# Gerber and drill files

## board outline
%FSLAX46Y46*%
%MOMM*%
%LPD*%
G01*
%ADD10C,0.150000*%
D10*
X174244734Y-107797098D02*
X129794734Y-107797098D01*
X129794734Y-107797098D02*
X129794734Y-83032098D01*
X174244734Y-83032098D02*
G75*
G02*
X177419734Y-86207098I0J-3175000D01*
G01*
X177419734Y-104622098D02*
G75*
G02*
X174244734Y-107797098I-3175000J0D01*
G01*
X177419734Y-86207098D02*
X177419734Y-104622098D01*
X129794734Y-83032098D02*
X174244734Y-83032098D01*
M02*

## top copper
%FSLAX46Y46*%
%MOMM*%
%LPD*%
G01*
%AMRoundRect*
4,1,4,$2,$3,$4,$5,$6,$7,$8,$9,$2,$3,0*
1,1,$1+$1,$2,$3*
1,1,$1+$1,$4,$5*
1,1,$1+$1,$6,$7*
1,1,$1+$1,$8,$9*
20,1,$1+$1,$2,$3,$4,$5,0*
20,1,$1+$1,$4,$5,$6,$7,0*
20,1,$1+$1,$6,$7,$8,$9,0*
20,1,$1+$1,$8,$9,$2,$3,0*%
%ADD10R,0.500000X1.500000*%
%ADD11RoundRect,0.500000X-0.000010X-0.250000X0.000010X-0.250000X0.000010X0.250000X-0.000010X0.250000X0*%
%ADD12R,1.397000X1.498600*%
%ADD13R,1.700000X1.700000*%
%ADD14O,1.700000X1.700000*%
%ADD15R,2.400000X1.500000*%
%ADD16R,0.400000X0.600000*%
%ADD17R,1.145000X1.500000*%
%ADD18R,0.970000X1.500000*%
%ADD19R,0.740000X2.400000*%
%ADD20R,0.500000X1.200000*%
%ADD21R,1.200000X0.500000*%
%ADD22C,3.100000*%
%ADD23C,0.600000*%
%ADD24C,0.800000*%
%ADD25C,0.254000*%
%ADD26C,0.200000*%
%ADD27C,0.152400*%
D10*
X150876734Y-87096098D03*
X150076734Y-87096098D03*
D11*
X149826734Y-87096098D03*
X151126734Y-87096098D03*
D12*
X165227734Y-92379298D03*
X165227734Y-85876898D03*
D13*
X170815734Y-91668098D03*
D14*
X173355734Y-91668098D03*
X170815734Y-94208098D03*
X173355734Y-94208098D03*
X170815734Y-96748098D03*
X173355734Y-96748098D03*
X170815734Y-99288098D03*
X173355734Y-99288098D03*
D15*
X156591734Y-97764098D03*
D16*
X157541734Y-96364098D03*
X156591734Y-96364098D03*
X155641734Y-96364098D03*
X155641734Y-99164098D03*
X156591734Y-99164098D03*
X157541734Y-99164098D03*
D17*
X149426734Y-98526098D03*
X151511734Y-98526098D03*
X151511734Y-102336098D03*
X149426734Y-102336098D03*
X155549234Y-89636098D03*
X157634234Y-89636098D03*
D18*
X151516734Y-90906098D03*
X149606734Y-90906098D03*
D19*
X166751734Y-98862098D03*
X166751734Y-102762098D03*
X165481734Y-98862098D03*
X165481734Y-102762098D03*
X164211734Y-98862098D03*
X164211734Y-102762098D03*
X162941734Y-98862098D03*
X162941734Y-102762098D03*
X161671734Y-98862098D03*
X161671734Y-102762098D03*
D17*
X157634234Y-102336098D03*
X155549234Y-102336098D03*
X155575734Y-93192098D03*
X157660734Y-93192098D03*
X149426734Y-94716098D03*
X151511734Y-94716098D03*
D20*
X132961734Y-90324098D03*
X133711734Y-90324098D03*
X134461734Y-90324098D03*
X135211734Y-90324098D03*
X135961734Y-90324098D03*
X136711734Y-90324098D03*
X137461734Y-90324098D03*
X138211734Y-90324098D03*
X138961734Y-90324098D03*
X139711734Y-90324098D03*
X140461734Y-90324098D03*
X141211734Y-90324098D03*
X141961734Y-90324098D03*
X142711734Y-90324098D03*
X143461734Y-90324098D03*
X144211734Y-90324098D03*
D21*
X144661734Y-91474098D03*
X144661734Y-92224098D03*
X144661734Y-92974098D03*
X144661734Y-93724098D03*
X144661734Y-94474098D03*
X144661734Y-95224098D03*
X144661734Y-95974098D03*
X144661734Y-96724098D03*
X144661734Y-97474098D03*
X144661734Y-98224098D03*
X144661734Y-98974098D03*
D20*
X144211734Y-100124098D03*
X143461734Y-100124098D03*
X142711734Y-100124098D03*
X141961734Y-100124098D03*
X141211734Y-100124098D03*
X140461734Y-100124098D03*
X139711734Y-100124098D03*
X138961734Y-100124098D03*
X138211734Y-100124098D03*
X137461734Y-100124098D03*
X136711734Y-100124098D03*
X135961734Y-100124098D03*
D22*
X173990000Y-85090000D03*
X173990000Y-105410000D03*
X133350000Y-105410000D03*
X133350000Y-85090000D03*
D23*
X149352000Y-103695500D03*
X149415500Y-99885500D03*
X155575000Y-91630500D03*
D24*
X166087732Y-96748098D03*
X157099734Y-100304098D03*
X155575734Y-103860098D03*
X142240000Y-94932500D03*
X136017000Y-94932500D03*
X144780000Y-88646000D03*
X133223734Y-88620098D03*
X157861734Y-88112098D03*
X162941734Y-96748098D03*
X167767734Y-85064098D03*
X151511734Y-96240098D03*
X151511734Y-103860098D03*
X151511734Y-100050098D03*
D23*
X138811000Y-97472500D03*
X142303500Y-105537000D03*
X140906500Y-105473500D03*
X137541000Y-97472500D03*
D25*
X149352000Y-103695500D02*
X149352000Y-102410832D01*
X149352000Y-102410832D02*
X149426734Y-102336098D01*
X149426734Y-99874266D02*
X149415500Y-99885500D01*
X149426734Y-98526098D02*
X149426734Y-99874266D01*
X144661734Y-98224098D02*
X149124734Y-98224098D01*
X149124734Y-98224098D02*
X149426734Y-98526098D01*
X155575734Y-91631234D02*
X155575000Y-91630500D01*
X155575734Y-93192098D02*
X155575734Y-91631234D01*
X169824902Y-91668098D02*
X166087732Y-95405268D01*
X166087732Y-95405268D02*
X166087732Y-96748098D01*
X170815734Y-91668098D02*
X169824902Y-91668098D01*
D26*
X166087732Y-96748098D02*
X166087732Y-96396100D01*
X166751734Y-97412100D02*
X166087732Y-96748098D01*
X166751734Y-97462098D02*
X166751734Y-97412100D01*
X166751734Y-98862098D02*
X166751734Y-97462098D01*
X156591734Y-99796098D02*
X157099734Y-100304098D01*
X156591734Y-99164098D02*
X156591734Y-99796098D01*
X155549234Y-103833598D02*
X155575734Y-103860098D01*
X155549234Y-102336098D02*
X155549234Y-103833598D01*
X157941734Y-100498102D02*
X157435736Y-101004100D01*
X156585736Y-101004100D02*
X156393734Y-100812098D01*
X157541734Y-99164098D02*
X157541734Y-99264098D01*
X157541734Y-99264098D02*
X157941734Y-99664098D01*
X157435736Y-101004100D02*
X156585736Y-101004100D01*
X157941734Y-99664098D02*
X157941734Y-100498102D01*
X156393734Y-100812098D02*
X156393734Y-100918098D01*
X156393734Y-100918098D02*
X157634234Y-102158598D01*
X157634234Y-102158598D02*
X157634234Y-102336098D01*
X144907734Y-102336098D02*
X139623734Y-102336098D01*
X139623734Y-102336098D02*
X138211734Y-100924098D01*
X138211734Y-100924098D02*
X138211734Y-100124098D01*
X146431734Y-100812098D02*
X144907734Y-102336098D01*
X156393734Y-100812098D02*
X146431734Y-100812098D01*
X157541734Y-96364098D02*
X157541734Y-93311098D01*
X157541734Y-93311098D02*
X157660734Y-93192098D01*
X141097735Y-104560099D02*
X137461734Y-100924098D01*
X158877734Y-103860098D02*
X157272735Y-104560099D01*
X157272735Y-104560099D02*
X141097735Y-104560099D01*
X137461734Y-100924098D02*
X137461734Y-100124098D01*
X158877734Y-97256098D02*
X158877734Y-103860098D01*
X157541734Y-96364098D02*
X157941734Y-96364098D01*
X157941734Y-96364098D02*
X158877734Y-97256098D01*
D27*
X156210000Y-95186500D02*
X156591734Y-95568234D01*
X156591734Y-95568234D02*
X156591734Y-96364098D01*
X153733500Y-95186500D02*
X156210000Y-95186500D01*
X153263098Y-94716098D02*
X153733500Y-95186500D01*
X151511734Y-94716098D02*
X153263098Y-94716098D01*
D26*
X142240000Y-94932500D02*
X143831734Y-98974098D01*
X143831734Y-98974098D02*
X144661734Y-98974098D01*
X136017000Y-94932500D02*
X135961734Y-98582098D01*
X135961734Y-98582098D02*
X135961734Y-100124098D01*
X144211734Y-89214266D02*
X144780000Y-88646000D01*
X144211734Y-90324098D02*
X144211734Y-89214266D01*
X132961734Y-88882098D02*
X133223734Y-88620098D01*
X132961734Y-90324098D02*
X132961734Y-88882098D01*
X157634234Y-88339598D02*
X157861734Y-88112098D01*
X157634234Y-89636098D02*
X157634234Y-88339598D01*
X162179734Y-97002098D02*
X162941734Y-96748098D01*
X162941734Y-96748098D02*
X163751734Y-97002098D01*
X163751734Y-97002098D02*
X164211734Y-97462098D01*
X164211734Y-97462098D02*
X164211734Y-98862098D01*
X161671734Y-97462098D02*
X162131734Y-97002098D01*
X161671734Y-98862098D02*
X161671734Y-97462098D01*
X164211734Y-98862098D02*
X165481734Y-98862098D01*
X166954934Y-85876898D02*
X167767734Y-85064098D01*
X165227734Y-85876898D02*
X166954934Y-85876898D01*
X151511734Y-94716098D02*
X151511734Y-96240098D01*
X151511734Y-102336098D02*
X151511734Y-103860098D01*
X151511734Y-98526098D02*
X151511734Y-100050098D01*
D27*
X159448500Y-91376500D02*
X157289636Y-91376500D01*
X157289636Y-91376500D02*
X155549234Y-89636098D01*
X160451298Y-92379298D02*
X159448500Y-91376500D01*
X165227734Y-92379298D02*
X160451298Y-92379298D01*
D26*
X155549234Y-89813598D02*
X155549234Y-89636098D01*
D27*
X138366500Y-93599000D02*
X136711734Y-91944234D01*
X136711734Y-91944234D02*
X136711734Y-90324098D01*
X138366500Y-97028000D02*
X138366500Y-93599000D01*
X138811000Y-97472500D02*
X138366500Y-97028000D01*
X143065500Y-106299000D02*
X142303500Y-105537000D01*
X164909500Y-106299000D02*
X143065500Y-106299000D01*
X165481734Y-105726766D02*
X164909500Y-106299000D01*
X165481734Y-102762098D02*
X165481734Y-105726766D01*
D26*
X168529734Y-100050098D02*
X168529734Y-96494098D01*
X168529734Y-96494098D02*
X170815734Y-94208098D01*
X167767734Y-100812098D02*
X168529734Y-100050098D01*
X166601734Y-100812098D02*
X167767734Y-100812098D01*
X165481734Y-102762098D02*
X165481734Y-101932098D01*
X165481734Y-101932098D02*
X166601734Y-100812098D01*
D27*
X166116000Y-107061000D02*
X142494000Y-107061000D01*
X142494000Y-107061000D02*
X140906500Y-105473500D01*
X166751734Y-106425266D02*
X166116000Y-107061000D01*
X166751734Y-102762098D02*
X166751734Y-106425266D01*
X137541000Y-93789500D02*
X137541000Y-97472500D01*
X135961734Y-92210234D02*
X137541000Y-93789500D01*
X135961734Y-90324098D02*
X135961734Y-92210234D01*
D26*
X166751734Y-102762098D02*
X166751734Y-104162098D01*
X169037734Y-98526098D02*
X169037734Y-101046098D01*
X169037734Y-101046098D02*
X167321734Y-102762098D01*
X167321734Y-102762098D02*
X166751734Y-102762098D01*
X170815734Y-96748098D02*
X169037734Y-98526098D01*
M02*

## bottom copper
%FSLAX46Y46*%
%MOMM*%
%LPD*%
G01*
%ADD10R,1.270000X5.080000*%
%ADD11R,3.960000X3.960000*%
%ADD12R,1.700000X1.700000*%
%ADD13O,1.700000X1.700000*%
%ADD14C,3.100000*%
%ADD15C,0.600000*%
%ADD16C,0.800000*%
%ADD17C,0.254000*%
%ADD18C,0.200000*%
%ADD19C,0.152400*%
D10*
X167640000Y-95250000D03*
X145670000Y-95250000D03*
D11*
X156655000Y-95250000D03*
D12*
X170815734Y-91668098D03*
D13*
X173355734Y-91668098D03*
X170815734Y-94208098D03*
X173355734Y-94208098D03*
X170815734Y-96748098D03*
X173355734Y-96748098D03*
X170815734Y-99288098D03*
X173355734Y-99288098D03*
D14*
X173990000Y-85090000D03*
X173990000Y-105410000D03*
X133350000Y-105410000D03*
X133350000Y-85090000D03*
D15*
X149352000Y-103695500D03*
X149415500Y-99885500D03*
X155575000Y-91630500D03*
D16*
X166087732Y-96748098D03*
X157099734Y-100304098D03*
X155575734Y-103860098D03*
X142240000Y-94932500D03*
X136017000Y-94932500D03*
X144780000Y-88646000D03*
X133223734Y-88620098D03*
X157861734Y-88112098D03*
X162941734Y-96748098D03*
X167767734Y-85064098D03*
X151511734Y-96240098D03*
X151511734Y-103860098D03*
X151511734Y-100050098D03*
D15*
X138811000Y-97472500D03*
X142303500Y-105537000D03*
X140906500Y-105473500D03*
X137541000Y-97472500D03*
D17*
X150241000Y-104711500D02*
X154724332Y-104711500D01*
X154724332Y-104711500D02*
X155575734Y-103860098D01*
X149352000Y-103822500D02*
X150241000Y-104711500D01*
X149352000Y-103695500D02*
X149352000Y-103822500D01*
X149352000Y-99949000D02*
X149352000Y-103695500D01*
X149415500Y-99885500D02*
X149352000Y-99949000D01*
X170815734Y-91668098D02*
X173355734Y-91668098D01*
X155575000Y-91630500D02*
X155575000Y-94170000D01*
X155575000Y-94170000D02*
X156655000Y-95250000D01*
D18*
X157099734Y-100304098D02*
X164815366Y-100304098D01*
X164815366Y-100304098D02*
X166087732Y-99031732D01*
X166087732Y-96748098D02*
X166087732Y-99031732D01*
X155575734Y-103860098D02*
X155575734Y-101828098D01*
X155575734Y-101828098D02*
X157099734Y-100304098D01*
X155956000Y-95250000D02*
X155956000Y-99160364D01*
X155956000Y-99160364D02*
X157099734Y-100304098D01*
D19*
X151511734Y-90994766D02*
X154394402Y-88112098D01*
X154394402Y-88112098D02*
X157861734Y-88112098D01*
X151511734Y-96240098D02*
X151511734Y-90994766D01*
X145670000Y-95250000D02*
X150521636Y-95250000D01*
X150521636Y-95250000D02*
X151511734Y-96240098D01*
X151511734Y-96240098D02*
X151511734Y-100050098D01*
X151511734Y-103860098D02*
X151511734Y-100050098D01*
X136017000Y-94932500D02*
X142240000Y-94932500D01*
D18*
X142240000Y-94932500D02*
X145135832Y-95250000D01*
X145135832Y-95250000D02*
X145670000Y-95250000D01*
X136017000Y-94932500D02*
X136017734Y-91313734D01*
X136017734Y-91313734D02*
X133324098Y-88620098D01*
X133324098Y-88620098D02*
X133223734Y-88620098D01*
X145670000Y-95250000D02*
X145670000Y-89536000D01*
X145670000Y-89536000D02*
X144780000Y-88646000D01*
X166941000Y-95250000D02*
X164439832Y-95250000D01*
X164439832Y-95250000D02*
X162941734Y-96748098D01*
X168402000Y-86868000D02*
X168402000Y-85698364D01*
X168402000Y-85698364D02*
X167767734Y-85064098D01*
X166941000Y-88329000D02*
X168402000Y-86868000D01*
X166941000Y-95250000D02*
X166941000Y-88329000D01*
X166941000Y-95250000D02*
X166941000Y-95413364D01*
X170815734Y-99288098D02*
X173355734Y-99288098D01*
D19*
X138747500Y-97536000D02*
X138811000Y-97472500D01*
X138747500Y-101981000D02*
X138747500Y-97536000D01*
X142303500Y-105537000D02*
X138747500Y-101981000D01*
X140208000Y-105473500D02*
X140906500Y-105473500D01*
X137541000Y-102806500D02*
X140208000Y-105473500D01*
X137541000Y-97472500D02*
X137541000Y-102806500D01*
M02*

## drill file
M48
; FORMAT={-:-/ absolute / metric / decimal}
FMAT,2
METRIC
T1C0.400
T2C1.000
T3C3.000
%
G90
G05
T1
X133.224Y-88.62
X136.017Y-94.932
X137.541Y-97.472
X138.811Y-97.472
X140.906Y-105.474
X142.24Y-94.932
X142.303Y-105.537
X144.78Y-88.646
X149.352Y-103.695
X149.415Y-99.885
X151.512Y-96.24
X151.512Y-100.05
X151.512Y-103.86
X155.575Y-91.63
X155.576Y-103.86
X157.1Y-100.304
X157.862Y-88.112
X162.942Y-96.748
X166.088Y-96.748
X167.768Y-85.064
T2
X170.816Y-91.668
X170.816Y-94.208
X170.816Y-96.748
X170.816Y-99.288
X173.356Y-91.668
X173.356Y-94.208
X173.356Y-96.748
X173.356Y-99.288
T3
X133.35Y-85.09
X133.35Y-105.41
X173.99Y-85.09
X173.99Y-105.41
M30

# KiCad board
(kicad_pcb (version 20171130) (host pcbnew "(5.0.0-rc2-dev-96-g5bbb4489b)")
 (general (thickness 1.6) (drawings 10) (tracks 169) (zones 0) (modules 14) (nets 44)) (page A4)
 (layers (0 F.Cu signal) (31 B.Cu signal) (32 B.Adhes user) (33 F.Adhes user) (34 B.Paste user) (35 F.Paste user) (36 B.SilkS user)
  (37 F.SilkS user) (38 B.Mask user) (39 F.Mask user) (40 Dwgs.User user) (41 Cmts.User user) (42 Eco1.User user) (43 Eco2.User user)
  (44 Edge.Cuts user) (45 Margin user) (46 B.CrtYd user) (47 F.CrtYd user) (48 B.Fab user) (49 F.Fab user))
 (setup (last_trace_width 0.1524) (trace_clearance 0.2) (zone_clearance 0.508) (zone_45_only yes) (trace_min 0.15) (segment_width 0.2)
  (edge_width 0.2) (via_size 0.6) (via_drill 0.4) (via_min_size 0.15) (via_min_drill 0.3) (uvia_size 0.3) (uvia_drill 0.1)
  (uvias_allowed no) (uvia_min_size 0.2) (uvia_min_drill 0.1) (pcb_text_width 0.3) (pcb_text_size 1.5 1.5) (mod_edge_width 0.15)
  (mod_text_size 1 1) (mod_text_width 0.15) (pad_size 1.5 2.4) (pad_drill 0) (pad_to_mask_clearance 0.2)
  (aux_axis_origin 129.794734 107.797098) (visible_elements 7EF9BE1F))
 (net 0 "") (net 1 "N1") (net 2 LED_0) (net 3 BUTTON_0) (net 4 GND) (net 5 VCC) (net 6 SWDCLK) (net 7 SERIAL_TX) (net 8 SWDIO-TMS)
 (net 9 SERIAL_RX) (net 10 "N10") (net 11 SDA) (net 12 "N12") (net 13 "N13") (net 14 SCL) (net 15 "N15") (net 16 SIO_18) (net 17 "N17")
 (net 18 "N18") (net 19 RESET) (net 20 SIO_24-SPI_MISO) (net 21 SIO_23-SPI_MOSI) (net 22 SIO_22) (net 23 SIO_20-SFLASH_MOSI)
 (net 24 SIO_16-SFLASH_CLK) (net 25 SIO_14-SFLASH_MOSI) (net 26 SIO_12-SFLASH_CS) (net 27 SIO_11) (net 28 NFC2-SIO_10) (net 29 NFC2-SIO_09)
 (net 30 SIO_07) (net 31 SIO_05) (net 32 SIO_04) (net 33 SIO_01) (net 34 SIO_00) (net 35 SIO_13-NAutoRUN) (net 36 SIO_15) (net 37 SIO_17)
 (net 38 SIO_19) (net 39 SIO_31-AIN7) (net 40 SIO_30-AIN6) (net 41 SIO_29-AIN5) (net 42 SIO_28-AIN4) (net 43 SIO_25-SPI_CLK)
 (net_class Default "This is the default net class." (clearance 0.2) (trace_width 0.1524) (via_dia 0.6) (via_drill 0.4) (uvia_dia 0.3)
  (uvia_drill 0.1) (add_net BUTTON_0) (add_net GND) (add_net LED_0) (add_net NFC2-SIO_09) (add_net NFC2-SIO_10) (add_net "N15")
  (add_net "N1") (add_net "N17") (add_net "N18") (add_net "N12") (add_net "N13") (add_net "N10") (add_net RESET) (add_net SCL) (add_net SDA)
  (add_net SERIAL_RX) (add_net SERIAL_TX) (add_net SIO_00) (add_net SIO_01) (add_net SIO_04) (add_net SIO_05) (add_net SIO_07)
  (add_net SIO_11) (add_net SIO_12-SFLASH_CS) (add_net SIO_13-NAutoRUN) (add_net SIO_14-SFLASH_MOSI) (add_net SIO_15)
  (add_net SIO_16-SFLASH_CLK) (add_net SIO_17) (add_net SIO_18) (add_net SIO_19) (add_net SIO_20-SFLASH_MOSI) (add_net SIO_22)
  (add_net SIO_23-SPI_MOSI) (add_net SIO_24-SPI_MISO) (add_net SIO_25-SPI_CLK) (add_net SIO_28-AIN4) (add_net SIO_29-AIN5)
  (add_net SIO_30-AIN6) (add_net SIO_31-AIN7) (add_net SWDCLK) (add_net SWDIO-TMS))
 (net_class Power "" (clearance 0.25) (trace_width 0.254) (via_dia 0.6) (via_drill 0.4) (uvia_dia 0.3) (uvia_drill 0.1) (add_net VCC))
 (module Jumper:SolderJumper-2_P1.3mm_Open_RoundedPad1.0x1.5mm (layer F.Cu) (at 150.476734 87.096098)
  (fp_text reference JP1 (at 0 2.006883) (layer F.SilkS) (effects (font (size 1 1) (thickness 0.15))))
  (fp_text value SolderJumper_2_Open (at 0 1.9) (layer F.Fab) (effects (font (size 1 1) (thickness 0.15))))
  (pad "" smd rect (at 0.4 0) (size 0.5 1.5) (layers F.Cu F.Mask))
  (pad "" smd rect (at -0.4 0) (size 0.5 1.5) (layers F.Cu F.Mask))
  (pad 1 smd roundrect (at -0.65 0) (size 1 1.5) (layers F.Cu F.Mask) (roundrect_rratio 0.5) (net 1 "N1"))
  (pad 2 smd roundrect (at 0.65 0) (size 1 1.5) (layers F.Cu F.Mask) (roundrect_rratio 0.5) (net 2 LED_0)))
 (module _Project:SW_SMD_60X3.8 (layer F.Cu) (at 165.227734 89.128098 270)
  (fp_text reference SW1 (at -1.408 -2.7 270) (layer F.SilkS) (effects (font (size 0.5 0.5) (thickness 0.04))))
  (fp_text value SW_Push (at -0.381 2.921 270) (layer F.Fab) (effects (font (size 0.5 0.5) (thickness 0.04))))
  (pad 2 smd rect (at 3.2512 0 270) (size 1.4986 1.397) (layers F.Cu F.Paste F.Mask) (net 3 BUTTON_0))
  (pad 1 smd rect (at -3.2512 0 270) (size 1.4986 1.397) (layers F.Cu F.Paste F.Mask) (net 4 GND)))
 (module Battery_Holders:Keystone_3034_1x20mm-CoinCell (layer B.Cu) (at 156.655 95.25 180)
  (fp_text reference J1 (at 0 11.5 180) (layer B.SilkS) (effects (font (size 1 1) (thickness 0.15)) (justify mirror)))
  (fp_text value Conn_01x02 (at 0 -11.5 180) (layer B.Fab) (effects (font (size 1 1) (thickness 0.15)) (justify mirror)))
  (pad 1 smd rect (at -10.985 0 180) (size 1.27 5.08) (layers B.Cu B.Paste B.Mask) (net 4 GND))
  (pad 1 smd rect (at 10.985 0 180) (size 1.27 5.08) (layers B.Cu B.Paste B.Mask) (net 4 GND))
  (pad 2 smd rect (at 0 0 180) (size 3.96 3.96) (layers B.Cu B.Paste B.Mask) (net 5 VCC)))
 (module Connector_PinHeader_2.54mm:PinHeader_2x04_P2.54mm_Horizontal (layer F.Cu) (at 170.815734 91.668098)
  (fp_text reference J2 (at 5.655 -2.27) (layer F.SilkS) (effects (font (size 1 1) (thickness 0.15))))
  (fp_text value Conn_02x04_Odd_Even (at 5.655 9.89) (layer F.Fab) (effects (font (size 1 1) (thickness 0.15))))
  (pad 1 thru_hole rect (at 0 0) (size 1.7 1.7) (drill 1) (layers *.Cu *.Mask) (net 5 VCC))
  (pad 2 thru_hole oval (at 2.54 0) (size 1.7 1.7) (drill 1) (layers *.Cu *.Mask) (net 5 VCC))
  (pad 3 thru_hole oval (at 0 2.54) (size 1.7 1.7) (drill 1) (layers *.Cu *.Mask) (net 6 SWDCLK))
  (pad 4 thru_hole oval (at 2.54 2.54) (size 1.7 1.7) (drill 1) (layers *.Cu *.Mask) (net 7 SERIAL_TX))
  (pad 5 thru_hole oval (at 0 5.08) (size 1.7 1.7) (drill 1) (layers *.Cu *.Mask) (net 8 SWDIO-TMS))
  (pad 6 thru_hole oval (at 2.54 5.08) (size 1.7 1.7) (drill 1) (layers *.Cu *.Mask) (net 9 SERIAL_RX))
  (pad 7 thru_hole oval (at 0 7.62) (size 1.7 1.7) (drill 1) (layers *.Cu *.Mask) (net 4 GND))
  (pad 8 thru_hole oval (at 2.54 7.62) (size 1.7 1.7) (drill 1) (layers *.Cu *.Mask) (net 4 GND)))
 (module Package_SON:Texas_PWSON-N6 (layer F.Cu) (at 156.591734 97.764098 270)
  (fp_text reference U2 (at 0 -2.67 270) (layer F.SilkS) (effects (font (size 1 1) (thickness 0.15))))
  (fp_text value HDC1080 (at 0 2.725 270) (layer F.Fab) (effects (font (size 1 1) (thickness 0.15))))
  (pad 7 smd rect (at 0 0 270) (size 1.5 2.4) (layers F.Cu F.Paste F.Mask) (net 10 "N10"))
  (pad 1 smd rect (at -1.4 -0.95 270) (size 0.6 0.4) (layers F.Cu F.Paste F.Mask) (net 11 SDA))
  (pad 2 smd rect (at -1.4 0 270) (size 0.6 0.4) (layers F.Cu F.Paste F.Mask) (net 4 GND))
  (pad 3 smd rect (at -1.4 0.95 270) (size 0.6 0.4) (layers F.Cu F.Paste F.Mask) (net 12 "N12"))
  (pad 4 smd rect (at 1.4 0.95 270) (size 0.6 0.4) (layers F.Cu F.Paste F.Mask) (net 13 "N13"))
  (pad 5 smd rect (at 1.4 0 270) (size 0.6 0.4) (layers F.Cu F.Paste F.Mask) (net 5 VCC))
  (pad 6 smd rect (at 1.4 -0.95 270) (size 0.6 0.4) (layers F.Cu F.Paste F.Mask) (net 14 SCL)))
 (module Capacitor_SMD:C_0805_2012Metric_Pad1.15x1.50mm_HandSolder (layer F.Cu) (at 150.469234 98.526098)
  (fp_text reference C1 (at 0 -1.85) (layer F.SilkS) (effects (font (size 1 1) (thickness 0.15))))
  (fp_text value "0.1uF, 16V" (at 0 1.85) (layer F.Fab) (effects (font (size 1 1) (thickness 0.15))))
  (pad 1 smd rect (at -1.0425 0) (size 1.145 1.5) (layers F.Cu F.Paste F.Mask) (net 5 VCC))
  (pad 2 smd rect (at 1.0425 0) (size 1.145 1.5) (layers F.Cu F.Paste F.Mask) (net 4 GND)))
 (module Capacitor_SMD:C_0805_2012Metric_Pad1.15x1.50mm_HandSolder (layer F.Cu) (at 150.469234 102.336098)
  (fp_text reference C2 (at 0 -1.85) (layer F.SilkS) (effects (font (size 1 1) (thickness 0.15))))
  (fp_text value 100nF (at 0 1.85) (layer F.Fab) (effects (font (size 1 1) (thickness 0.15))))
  (pad 2 smd rect (at 1.0425 0) (size 1.145 1.5) (layers F.Cu F.Paste F.Mask) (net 4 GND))
  (pad 1 smd rect (at -1.0425 0) (size 1.145 1.5) (layers F.Cu F.Paste F.Mask) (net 5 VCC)))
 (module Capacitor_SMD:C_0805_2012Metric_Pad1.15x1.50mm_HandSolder (layer F.Cu) (at 156.591734 89.636098)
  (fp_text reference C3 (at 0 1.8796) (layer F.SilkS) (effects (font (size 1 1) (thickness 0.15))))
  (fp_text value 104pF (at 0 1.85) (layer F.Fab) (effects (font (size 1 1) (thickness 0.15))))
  (pad 1 smd rect (at -1.0425 0) (size 1.145 1.5) (layers F.Cu F.Paste F.Mask) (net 3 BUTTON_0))
  (pad 2 smd rect (at 1.0425 0) (size 1.145 1.5) (layers F.Cu F.Paste F.Mask) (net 4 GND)))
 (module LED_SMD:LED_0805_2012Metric (layer F.Cu) (at 150.561734 90.906098 180)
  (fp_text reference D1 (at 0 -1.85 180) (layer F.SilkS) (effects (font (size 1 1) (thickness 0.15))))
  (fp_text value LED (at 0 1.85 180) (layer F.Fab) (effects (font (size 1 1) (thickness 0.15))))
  (pad 1 smd rect (at -0.955 0 180) (size 0.97 1.5) (layers F.Cu F.Paste F.Mask) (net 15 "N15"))
  (pad 2 smd rect (at 0.955 0 180) (size 0.97 1.5) (layers F.Cu F.Paste F.Mask) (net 1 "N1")))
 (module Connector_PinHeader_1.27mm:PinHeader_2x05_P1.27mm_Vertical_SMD (layer F.Cu) (at 164.211734 100.812098 270)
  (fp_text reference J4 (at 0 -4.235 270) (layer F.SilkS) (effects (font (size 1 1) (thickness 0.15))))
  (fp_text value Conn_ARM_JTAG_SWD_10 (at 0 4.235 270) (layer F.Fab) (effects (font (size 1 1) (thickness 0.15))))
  (pad 1 smd rect (at -1.95 -2.54 270) (size 2.4 0.74) (layers F.Cu F.Paste F.Mask) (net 5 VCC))
  (pad 2 smd rect (at 1.95 -2.54 270) (size 2.4 0.74) (layers F.Cu F.Paste F.Mask) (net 8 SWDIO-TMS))
  (pad 3 smd rect (at -1.95 -1.27 270) (size 2.4 0.74) (layers F.Cu F.Paste F.Mask) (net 4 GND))
  (pad 4 smd rect (at 1.95 -1.27 270) (size 2.4 0.74) (layers F.Cu F.Paste F.Mask) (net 6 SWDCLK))
  (pad 5 smd rect (at -1.95 0 270) (size 2.4 0.74) (layers F.Cu F.Paste F.Mask) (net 4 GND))
  (pad 6 smd rect (at 1.95 0 270) (size 2.4 0.74) (layers F.Cu F.Paste F.Mask) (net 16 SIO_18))
  (pad 7 smd rect (at -1.95 1.27 270) (size 2.4 0.74) (layers F.Cu F.Paste F.Mask) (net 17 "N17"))
  (pad 8 smd rect (at 1.95 1.27 270) (size 2.4 0.74) (layers F.Cu F.Paste F.Mask) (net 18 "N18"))
  (pad 9 smd rect (at -1.95 2.54 270) (size 2.4 0.74) (layers F.Cu F.Paste F.Mask) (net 4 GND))
  (pad 10 smd rect (at 1.95 2.54 270) (size 2.4 0.74) (layers F.Cu F.Paste F.Mask) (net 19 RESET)))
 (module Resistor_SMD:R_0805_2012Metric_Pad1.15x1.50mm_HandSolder (layer F.Cu) (at 156.591734 102.336098)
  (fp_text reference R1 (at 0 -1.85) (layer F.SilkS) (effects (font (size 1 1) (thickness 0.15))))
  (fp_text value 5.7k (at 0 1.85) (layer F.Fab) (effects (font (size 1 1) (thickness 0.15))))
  (pad 2 smd rect (at 1.0425 0) (size 1.145 1.5) (layers F.Cu F.Paste F.Mask) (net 14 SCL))
  (pad 1 smd rect (at -1.0425 0) (size 1.145 1.5) (layers F.Cu F.Paste F.Mask) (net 5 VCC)))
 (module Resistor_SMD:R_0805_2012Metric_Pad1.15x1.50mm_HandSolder (layer F.Cu) (at 156.618234 93.192098)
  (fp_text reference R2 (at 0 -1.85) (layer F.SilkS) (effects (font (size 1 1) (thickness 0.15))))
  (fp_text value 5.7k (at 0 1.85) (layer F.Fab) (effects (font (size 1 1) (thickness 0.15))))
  (pad 1 smd rect (at -1.0425 0) (size 1.145 1.5) (layers F.Cu F.Paste F.Mask) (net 5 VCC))
  (pad 2 smd rect (at 1.0425 0) (size 1.145 1.5) (layers F.Cu F.Paste F.Mask) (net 11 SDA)))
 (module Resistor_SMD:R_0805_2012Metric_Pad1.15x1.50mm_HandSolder (layer F.Cu) (at 150.469234 94.716098)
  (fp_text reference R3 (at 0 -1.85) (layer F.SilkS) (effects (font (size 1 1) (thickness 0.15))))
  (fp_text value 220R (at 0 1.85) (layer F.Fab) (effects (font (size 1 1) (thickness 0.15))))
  (pad 1 smd rect (at -1.0425 0) (size 1.145 1.5) (layers F.Cu F.Paste F.Mask) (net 15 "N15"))
  (pad 2 smd rect (at 1.0425 0) (size 1.145 1.5) (layers F.Cu F.Paste F.Mask) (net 4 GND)))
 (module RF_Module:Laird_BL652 (layer F.Cu) (at 138.811734 95.224098)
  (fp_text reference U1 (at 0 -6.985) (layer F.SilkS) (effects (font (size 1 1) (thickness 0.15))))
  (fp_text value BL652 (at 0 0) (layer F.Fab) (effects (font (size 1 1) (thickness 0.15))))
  (pad 1 smd rect (at -5.85 -4.9 90) (size 1.2 0.5) (layers F.Cu F.Paste F.Mask) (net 4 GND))
  (pad 2 smd rect (at -5.1 -4.9 90) (size 1.2 0.5) (layers F.Cu F.Paste F.Mask) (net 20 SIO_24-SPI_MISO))
  (pad 3 smd rect (at -4.35 -4.9 90) (size 1.2 0.5) (layers F.Cu F.Paste F.Mask) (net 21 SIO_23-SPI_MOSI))
  (pad 4 smd rect (at -3.6 -4.9 90) (size 1.2 0.5) (layers F.Cu F.Paste F.Mask) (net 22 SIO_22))
  (pad 5 smd rect (at -2.85 -4.9 90) (size 1.2 0.5) (layers F.Cu F.Paste F.Mask) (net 8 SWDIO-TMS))
  (pad 6 smd rect (at -2.1 -4.9 90) (size 1.2 0.5) (layers F.Cu F.Paste F.Mask) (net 6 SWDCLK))
  (pad 7 smd rect (at -1.35 -4.9 90) (size 1.2 0.5) (layers F.Cu F.Paste F.Mask) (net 19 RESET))
  (pad 8 smd rect (at -0.6 -4.9 90) (size 1.2 0.5) (layers F.Cu F.Paste F.Mask) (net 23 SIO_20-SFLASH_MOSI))
  (pad 9 smd rect (at 0.15 -4.9 90) (size 1.2 0.5) (layers F.Cu F.Paste F.Mask) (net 16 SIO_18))
  (pad 10 smd rect (at 0.9 -4.9 90) (size 1.2 0.5) (layers F.Cu F.Paste F.Mask) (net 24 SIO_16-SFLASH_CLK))
  (pad 11 smd rect (at 1.65 -4.9 90) (size 1.2 0.5) (layers F.Cu F.Paste F.Mask) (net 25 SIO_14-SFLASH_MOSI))
  (pad 12 smd rect (at 2.4 -4.9 90) (size 1.2 0.5) (layers F.Cu F.Paste F.Mask) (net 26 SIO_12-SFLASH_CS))
  (pad 13 smd rect (at 3.15 -4.9 90) (size 1.2 0.5) (layers F.Cu F.Paste F.Mask) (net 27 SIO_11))
  (pad 14 smd rect (at 3.9 -4.9 90) (size 1.2 0.5) (layers F.Cu F.Paste F.Mask) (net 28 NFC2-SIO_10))
  (pad 15 smd rect (at 4.65 -4.9 90) (size 1.2 0.5) (layers F.Cu F.Paste F.Mask) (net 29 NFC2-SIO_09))
  (pad 16 smd rect (at 5.4 -4.9 90) (size 1.2 0.5) (layers F.Cu F.Paste F.Mask) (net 4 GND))
  (pad 17 smd rect (at 5.85 -3.75) (size 1.2 0.5) (layers F.Cu F.Paste F.Mask) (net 7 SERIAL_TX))
  (pad 18 smd rect (at 5.85 -3) (size 1.2 0.5) (layers F.Cu F.Paste F.Mask) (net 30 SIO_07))
  (pad 19 smd rect (at 5.85 -2.25) (size 1.2 0.5) (layers F.Cu F.Paste F.Mask) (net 9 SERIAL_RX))
  (pad 20 smd rect (at 5.85 -1.5) (size 1.2 0.5) (layers F.Cu F.Paste F.Mask) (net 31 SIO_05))
  (pad 21 smd rect (at 5.85 -0.75) (size 1.2 0.5) (layers F.Cu F.Paste F.Mask) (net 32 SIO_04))
  (pad 22 smd rect (at 5.85 0) (size 1.2 0.5) (layers F.Cu F.Paste F.Mask) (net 3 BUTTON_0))
  (pad 23 smd rect (at 5.85 0.75) (size 1.2 0.5) (layers F.Cu F.Paste F.Mask) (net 2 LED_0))
  (pad 24 smd rect (at 5.85 1.5) (size 1.2 0.5) (layers F.Cu F.Paste F.Mask) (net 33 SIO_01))
  (pad 25 smd rect (at 5.85 2.25) (size 1.2 0.5) (layers F.Cu F.Paste F.Mask) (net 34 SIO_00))
  (pad 26 smd rect (at 5.85 3) (size 1.2 0.5) (layers F.Cu F.Paste F.Mask) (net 5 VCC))
  (pad 27 smd rect (at 5.85 3.75) (size 1.2 0.5) (layers F.Cu F.Paste F.Mask) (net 4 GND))
  (pad 28 smd rect (at 5.4 4.9 90) (size 1.2 0.5) (layers F.Cu F.Paste F.Mask) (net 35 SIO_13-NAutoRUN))
  (pad 29 smd rect (at 4.65 4.9 90) (size 1.2 0.5) (layers F.Cu F.Paste F.Mask) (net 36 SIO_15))
  (pad 30 smd rect (at 3.9 4.9 90) (size 1.2 0.5) (layers F.Cu F.Paste F.Mask) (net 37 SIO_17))
  (pad 31 smd rect (at 3.15 4.9 90) (size 1.2 0.5) (layers F.Cu F.Paste F.Mask) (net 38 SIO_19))
  (pad 32 smd rect (at 2.4 4.9 90) (size 1.2 0.5) (layers F.Cu F.Paste F.Mask) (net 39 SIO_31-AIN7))
  (pad 33 smd rect (at 1.65 4.9 90) (size 1.2 0.5) (layers F.Cu F.Paste F.Mask) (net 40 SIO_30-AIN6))
  (pad 34 smd rect (at 0.9 4.9 90) (size 1.2 0.5) (layers F.Cu F.Paste F.Mask) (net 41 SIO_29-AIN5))
  (pad 35 smd rect (at 0.15 4.9 90) (size 1.2 0.5) (layers F.Cu F.Paste F.Mask) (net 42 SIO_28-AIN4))
  (pad 36 smd rect (at -0.6 4.9 90) (size 1.2 0.5) (layers F.Cu F.Paste F.Mask) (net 14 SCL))
  (pad 37 smd rect (at -1.35 4.9 90) (size 1.2 0.5) (layers F.Cu F.Paste F.Mask) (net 11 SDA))
  (pad 38 smd rect (at -2.1 4.9 90) (size 1.2 0.5) (layers F.Cu F.Paste F.Mask) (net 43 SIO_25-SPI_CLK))
  (pad 39 smd rect (at -2.85 4.9 90) (size 1.2 0.5) (layers F.Cu F.Paste F.Mask) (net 4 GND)))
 (gr_line (start 174.244734 107.797098) (end 129.794734 107.797098) (layer Edge.Cuts) (width 0.15))
 (gr_line (start 129.794734 107.797098) (end 129.794734 83.032098) (layer Edge.Cuts) (width 0.15))
 (gr_arc (start 174.244734 86.207098) (end 177.419734 86.207098) (angle -90) (layer Edge.Cuts) (width 0.15))
 (gr_arc (start 174.244734 104.622098) (end 174.244734 107.797098) (angle -90) (layer Edge.Cuts) (width 0.15))
 (gr_line (start 177.419734 86.207098) (end 177.419734 104.622098) (layer Edge.Cuts) (width 0.15))
 (gr_line (start 129.794734 83.032098) (end 174.244734 83.032098) (layer Edge.Cuts) (width 0.15))
 (via (at 173.99 85.09) (size 3.1) (drill 3) (layers F.Cu B.Cu) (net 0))
 (via (at 173.99 105.41) (size 3.1) (drill 3) (layers F.Cu B.Cu) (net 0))
 (via (at 133.35 105.41) (size 3.1) (drill 3) (layers F.Cu B.Cu) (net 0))
 (via (at 133.35 85.09) (size 3.1) (drill 3) (layers F.Cu B.Cu) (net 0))
 (segment (start 150.241 104.7115) (end 154.724332 104.7115) (width 0.254) (layer B.Cu) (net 5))
 (segment (start 154.724332 104.7115) (end 155.575734 103.860098) (width 0.254) (layer B.Cu) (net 5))
 (segment (start 149.352 103.8225) (end 150.241 104.7115) (width 0.254) (layer B.Cu) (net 5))
 (segment (start 149.352 103.6955) (end 149.352 103.8225) (width 0.254) (layer B.Cu) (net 5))
 (segment (start 149.352 103.6955) (end 149.352 102.410832) (width 0.254) (layer F.Cu) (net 5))
 (segment (start 149.352 102.410832) (end 149.426734 102.336098) (width 0.254) (layer F.Cu) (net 5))
 (segment (start 149.352 99.949) (end 149.352 103.6955) (width 0.254) (layer B.Cu) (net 5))
 (segment (start 149.4155 99.8855) (end 149.352 99.949) (width 0.254) (layer B.Cu) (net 5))
 (via (at 149.352 103.6955) (size 0.6) (drill 0.4) (layers F.Cu B.Cu) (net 5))
 (segment (start 149.426734 99.874266) (end 149.4155 99.8855) (width 0.254) (layer F.Cu) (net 5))
 (segment (start 149.426734 98.526098) (end 149.426734 99.874266) (width 0.254) (layer F.Cu) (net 5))
 (via (at 149.4155 99.8855) (size 0.6) (drill 0.4) (layers F.Cu B.Cu) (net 5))
 (segment (start 170.815734 91.668098) (end 173.355734 91.668098) (width 0.254) (layer B.Cu) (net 5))
 (segment (start 155.575 91.6305) (end 155.575 94.17) (width 0.254) (layer B.Cu) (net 5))
 (segment (start 155.575 94.17) (end 156.655 95.25) (width 0.254) (layer B.Cu) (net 5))
 (segment (start 144.661734 98.224098) (end 149.124734 98.224098) (width 0.254) (layer F.Cu) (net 5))
 (segment (start 149.124734 98.224098) (end 149.426734 98.526098) (width 0.254) (layer F.Cu) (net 5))
 (segment (start 155.575734 91.631234) (end 155.575 91.6305) (width 0.254) (layer F.Cu) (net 5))
 (segment (start 155.575734 93.192098) (end 155.575734 91.631234) (width 0.254) (layer F.Cu) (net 5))
 (via (at 155.575 91.6305) (size 0.6) (drill 0.4) (layers F.Cu B.Cu) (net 5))
 (segment (start 169.824902 91.668098) (end 166.087732 95.405268) (width 0.254) (layer F.Cu) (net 5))
 (segment (start 166.087732 95.405268) (end 166.087732 96.748098) (width 0.254) (layer F.Cu) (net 5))
 (segment (start 170.815734 91.668098) (end 169.824902 91.668098) (width 0.254) (layer F.Cu) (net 5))
 (segment (start 166.087732 96.748098) (end 166.087732 96.3961) (width 0.2) (layer F.Cu) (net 5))
 (segment (start 157.099734 100.304098) (end 164.815366 100.304098) (width 0.2) (layer B.Cu) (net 5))
 (segment (start 164.815366 100.304098) (end 166.087732 99.031732) (width 0.2) (layer B.Cu) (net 5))
 (segment (start 166.087732 96.748098) (end 166.087732 99.031732) (width 0.2) (layer B.Cu) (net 5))
 (segment (start 155.575734 103.860098) (end 155.575734 101.828098) (width 0.2) (layer B.Cu) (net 5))
 (segment (start 155.575734 101.828098) (end 157.099734 100.304098) (width 0.2) (layer B.Cu) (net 5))
 (segment (start 155.956 95.25) (end 155.956 99.160364) (width 0.2) (layer B.Cu) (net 5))
 (segment (start 155.956 99.160364) (end 157.099734 100.304098) (width 0.2) (layer B.Cu) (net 5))
 (segment (start 166.751734 97.4121) (end 166.087732 96.748098) (width 0.2) (layer F.Cu) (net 5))
 (segment (start 166.751734 97.462098) (end 166.751734 97.4121) (width 0.2) (layer F.Cu) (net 5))
 (via (at 166.087732 96.748098) (size 0.8) (drill 0.4) (layers F.Cu B.Cu) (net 5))
 (segment (start 166.751734 98.862098) (end 166.751734 97.462098) (width 0.2) (layer F.Cu) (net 5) (status 10))
 (segment (start 156.591734 99.796098) (end 157.099734 100.304098) (width 0.2) (layer F.Cu) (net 5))
 (segment (start 156.591734 99.164098) (end 156.591734 99.796098) (width 0.2) (layer F.Cu) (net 5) (status 10))
 (via (at 157.099734 100.304098) (size 0.8) (drill 0.4) (layers F.Cu B.Cu) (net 5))
 (segment (start 155.549234 103.833598) (end 155.575734 103.860098) (width 0.2) (layer F.Cu) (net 5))
 (segment (start 155.549234 102.336098) (end 155.549234 103.833598) (width 0.2) (layer F.Cu) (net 5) (status 10))
 (via (at 155.575734 103.860098) (size 0.8) (drill 0.4) (layers F.Cu B.Cu) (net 5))
 (segment (start 157.941734 100.498102) (end 157.435736 101.0041) (width 0.2) (layer F.Cu) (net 14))
 (segment (start 156.585736 101.0041) (end 156.393734 100.812098) (width 0.2) (layer F.Cu) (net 14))
 (segment (start 157.541734 99.164098) (end 157.541734 99.264098) (width 0.2) (layer F.Cu) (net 14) (status 30))
 (segment (start 157.541734 99.264098) (end 157.941734 99.664098) (width 0.2) (layer F.Cu) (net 14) (status 10))
 (segment (start 157.435736 101.0041) (end 156.585736 101.0041) (width 0.2) (layer F.Cu) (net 14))
 (segment (start 157.941734 99.664098) (end 157.941734 100.498102) (width 0.2) (layer F.Cu) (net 14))
 (segment (start 156.393734 100.812098) (end 156.393734 100.918098) (width 0.2) (layer F.Cu) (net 14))
 (segment (start 156.393734 100.918098) (end 157.634234 102.158598) (width 0.2) (layer F.Cu) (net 14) (status 20))
 (segment (start 157.634234 102.158598) (end 157.634234 102.336098) (width 0.2) (layer F.Cu) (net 14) (status 30))
 (segment (start 144.907734 102.336098) (end 139.623734 102.336098) (width 0.2) (layer F.Cu) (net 14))
 (segment (start 139.623734 102.336098) (end 138.211734 100.924098) (width 0.2) (layer F.Cu) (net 14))
 (segment (start 138.211734 100.924098) (end 138.211734 100.124098) (width 0.2) (layer F.Cu) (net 14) (status 20))
 (segment (start 146.431734 100.812098) (end 144.907734 102.336098) (width 0.2) (layer F.Cu) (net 14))
 (segment (start 156.393734 100.812098) (end 146.431734 100.812098) (width 0.2) (layer F.Cu) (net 14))
 (segment (start 157.541734 96.364098) (end 157.541734 93.311098) (width 0.2) (layer F.Cu) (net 11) (status 30))
 (segment (start 157.541734 93.311098) (end 157.660734 93.192098) (width 0.2) (layer F.Cu) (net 11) (status 30))
 (segment (start 141.097735 104.560099) (end 137.461734 100.924098) (width 0.2) (layer F.Cu) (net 11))
 (segment (start 158.877734 103.860098) (end 157.272735 104.560099) (width 0.2) (layer F.Cu) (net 11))
 (segment (start 157.272735 104.560099) (end 141.097735 104.560099) (width 0.2) (layer F.Cu) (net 11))
 (segment (start 137.461734 100.924098) (end 137.461734 100.124098) (width 0.2) (layer F.Cu) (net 11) (status 20))
 (segment (start 158.877734 97.256098) (end 158.877734 103.860098) (width 0.2) (layer F.Cu) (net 11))
 (segment (start 157.541734 96.364098) (end 157.941734 96.364098) (width 0.2) (layer F.Cu) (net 11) (status 10))
 (segment (start 157.941734 96.364098) (end 158.877734 97.256098) (width 0.2) (layer F.Cu) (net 11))
 (segment (start 151.511734 90.994766) (end 154.394402 88.112098) (width 0.1524) (layer B.Cu) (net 4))
 (segment (start 154.394402 88.112098) (end 157.861734 88.112098) (width 0.1524) (layer B.Cu) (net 4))
 (segment (start 151.511734 96.240098) (end 151.511734 90.994766) (width 0.1524) (layer B.Cu) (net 4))
 (segment (start 145.67 95.25) (end 150.521636 95.25) (width 0.1524) (layer B.Cu) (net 4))
 (segment (start 150.521636 95.25) (end 151.511734 96.240098) (width 0.1524) (layer B.Cu) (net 4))
 (segment (start 156.21 95.1865) (end 156.591734 95.568234) (width 0.1524) (layer F.Cu) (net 4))
 (segment (start 156.591734 95.568234) (end 156.591734 96.364098) (width 0.1524) (layer F.Cu) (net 4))
 (segment (start 153.7335 95.1865) (end 156.21 95.1865) (width 0.1524) (layer F.Cu) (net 4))
 (segment (start 153.263098 94.716098) (end 153.7335 95.1865) (width 0.1524) (layer F.Cu) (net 4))
 (segment (start 151.511734 94.716098) (end 153.263098 94.716098) (width 0.1524) (layer F.Cu) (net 4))
 (segment (start 151.511734 96.240098) (end 151.511734 100.050098) (width 0.1524) (layer B.Cu) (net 4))
 (segment (start 151.511734 103.860098) (end 151.511734 100.050098) (width 0.1524) (layer B.Cu) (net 4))
 (segment (start 136.017 94.9325) (end 142.24 94.9325) (width 0.1524) (layer B.Cu) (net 4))
 (segment (start 142.24 94.9325) (end 143.831734 98.974098) (width 0.2) (layer F.Cu) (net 4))
 (segment (start 143.831734 98.974098) (end 144.661734 98.974098) (width 0.2) (layer F.Cu) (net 4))
 (segment (start 142.24 94.9325) (end 145.135832 95.25) (width 0.2) (layer B.Cu) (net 4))
 (segment (start 145.135832 95.25) (end 145.67 95.25) (width 0.2) (layer B.Cu) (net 4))
 (via (at 142.24 94.9325) (size 0.8) (drill 0.4) (layers F.Cu B.Cu) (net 4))
 (segment (start 136.017 94.9325) (end 135.961734 98.582098) (width 0.2) (layer F.Cu) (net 4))
 (segment (start 135.961734 98.582098) (end 135.961734 100.124098) (width 0.2) (layer F.Cu) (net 4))
 (segment (start 136.017 94.9325) (end 136.017734 91.313734) (width 0.2) (layer B.Cu) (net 4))
 (segment (start 136.017734 91.313734) (end 133.324098 88.620098) (width 0.2) (layer B.Cu) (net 4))
 (segment (start 133.324098 88.620098) (end 133.223734 88.620098) (width 0.2) (layer B.Cu) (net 4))
 (via (at 136.017 94.9325) (size 0.8) (drill 0.4) (layers F.Cu B.Cu) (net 4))
 (segment (start 145.67 95.25) (end 145.67 89.536) (width 0.2) (layer B.Cu) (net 4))
 (segment (start 145.67 89.536) (end 144.78 88.646) (width 0.2) (layer B.Cu) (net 4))
 (segment (start 144.211734 89.214266) (end 144.78 88.646) (width 0.2) (layer F.Cu) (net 4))
 (segment (start 144.211734 90.324098) (end 144.211734 89.214266) (width 0.2) (layer F.Cu) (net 4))
 (via (at 144.78 88.646) (size 0.8) (drill 0.4) (layers F.Cu B.Cu) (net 4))
 (segment (start 166.941 95.25) (end 164.439832 95.25) (width 0.2) (layer B.Cu) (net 4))
 (segment (start 164.439832 95.25) (end 162.941734 96.748098) (width 0.2) (layer B.Cu) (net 4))
 (segment (start 168.402 86.868) (end 168.402 85.698364) (width 0.2) (layer B.Cu) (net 4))
 (segment (start 168.402 85.698364) (end 167.767734 85.064098) (width 0.2) (layer B.Cu) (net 4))
 (segment (start 166.941 88.329) (end 168.402 86.868) (width 0.2) (layer B.Cu) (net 4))
 (segment (start 166.941 95.25) (end 166.941 88.329) (width 0.2) (layer B.Cu) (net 4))
 (segment (start 166.941 95.25) (end 166.941 95.413364) (width 0.2) (layer B.Cu) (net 4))
 (segment (start 132.961734 88.882098) (end 133.223734 88.620098) (width 0.2) (layer F.Cu) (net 4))
 (segment (start 132.961734 90.324098) (end 132.961734 88.882098) (width 0.2) (layer F.Cu) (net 4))
 (via (at 133.223734 88.620098) (size 0.8) (drill 0.4) (layers F.Cu B.Cu) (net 4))
 (segment (start 157.634234 88.339598) (end 157.861734 88.112098) (width 0.2) (layer F.Cu) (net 4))
 (segment (start 157.634234 89.636098) (end 157.634234 88.339598) (width 0.2) (layer F.Cu) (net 4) (status 10))
 (via (at 157.861734 88.112098) (size 0.8) (drill 0.4) (layers F.Cu B.Cu) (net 4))
 (segment (start 162.179734 97.002098) (end 162.941734 96.748098) (width 0.2) (layer F.Cu) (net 4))
 (segment (start 162.941734 96.748098) (end 163.751734 97.002098) (width 0.2) (layer F.Cu) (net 4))
 (segment (start 163.751734 97.002098) (end 164.211734 97.462098) (width 0.2) (layer F.Cu) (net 4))
 (segment (start 164.211734 97.462098) (end 164.211734 98.862098) (width 0.2) (layer F.Cu) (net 4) (status 20))
 (via (at 162.941734 96.748098) (size 0.8) (drill 0.4) (layers F.Cu B.Cu) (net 4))
 (segment (start 161.671734 97.462098) (end 162.131734 97.002098) (width 0.2) (layer F.Cu) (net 4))
 (segment (start 161.671734 98.862098) (end 161.671734 97.462098) (width 0.2) (layer F.Cu) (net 4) (status 10))
 (segment (start 170.815734 99.288098) (end 173.355734 99.288098) (width 0.2) (layer B.Cu) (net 4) (status 30))
 (segment (start 164.211734 98.862098) (end 165.481734 98.862098) (width 0.2) (layer F.Cu) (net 4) (status 30))
 (segment (start 166.954934 85.876898) (end 167.767734 85.064098) (width 0.2) (layer F.Cu) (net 4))
 (segment (start 165.227734 85.876898) (end 166.954934 85.876898) (width 0.2) (layer F.Cu) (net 4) (status 10))
 (via (at 167.767734 85.064098) (size 0.8) (drill 0.4) (layers F.Cu B.Cu) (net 4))
 (segment (start 151.511734 94.716098) (end 151.511734 96.240098) (width 0.2) (layer F.Cu) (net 4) (status 10))
 (via (at 151.511734 96.240098) (size 0.8) (drill 0.4) (layers F.Cu B.Cu) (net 4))
 (via (at 151.511734 103.860098) (size 0.8) (drill 0.4) (layers F.Cu B.Cu) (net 4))
 (segment (start 151.511734 102.336098) (end 151.511734 103.860098) (width 0.2) (layer F.Cu) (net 4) (status 10))
 (via (at 151.511734 100.050098) (size 0.8) (drill 0.4) (layers F.Cu B.Cu) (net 4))
 (segment (start 151.511734 98.526098) (end 151.511734 100.050098) (width 0.2) (layer F.Cu) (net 4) (status 10))
 (segment (start 159.4485 91.3765) (end 157.289636 91.3765) (width 0.1524) (layer F.Cu) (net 3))
 (segment (start 157.289636 91.3765) (end 155.549234 89.636098) (width 0.1524) (layer F.Cu) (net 3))
 (segment (start 160.451298 92.379298) (end 159.4485 91.3765) (width 0.1524) (layer F.Cu) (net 3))
 (segment (start 165.227734 92.379298) (end 160.451298 92.379298) (width 0.1524) (layer F.Cu) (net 3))
 (segment (start 155.549234 89.813598) (end 155.549234 89.636098) (width 0.2) (layer F.Cu) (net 3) (status 30))
 (segment (start 138.3665 93.599) (end 136.711734 91.944234) (width 0.1524) (layer F.Cu) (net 6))
 (segment (start 136.711734 91.944234) (end 136.711734 90.324098) (width 0.1524) (layer F.Cu) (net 6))
 (segment (start 138.3665 97.028) (end 138.3665 93.599) (width 0.1524) (layer F.Cu) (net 6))
 (segment (start 138.811 97.4725) (end 138.3665 97.028) (width 0.1524) (layer F.Cu) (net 6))
 (segment (start 138.7475 97.536) (end 138.811 97.4725) (width 0.1524) (layer B.Cu) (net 6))
 (segment (start 138.7475 101.981) (end 138.7475 97.536) (width 0.1524) (layer B.Cu) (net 6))
 (via (at 138.811 97.4725) (size 0.6) (drill 0.4) (layers F.Cu B.Cu) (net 6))
 (segment (start 142.3035 105.537) (end 138.7475 101.981) (width 0.1524) (layer B.Cu) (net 6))
 (segment (start 143.0655 106.299) (end 142.3035 105.537) (width 0.1524) (layer F.Cu) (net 6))
 (segment (start 164.9095 106.299) (end 143.0655 106.299) (width 0.1524) (layer F.Cu) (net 6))
 (via (at 142.3035 105.537) (size 0.6) (drill 0.4) (layers F.Cu B.Cu) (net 6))
 (segment (start 165.481734 105.726766) (end 164.9095 106.299) (width 0.1524) (layer F.Cu) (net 6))
 (segment (start 165.481734 102.762098) (end 165.481734 105.726766) (width 0.1524) (layer F.Cu) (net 6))
 (segment (start 168.529734 100.050098) (end 168.529734 96.494098) (width 0.2) (layer F.Cu) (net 6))
 (segment (start 168.529734 96.494098) (end 170.815734 94.208098) (width 0.2) (layer F.Cu) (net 6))
 (segment (start 167.767734 100.812098) (end 168.529734 100.050098) (width 0.2) (layer F.Cu) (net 6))
 (segment (start 166.601734 100.812098) (end 167.767734 100.812098) (width 0.2) (layer F.Cu) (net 6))
 (segment (start 165.481734 102.762098) (end 165.481734 101.932098) (width 0.2) (layer F.Cu) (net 6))
 (segment (start 165.481734 101.932098) (end 166.601734 100.812098) (width 0.2) (layer F.Cu) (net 6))
 (segment (start 166.116 107.061) (end 142.494 107.061) (width 0.1524) (layer F.Cu) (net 8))
 (segment (start 142.494 107.061) (end 140.9065 105.4735) (width 0.1524) (layer F.Cu) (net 8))
 (segment (start 166.751734 106.425266) (end 166.116 107.061) (width 0.1524) (layer F.Cu) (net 8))
 (segment (start 166.751734 102.762098) (end 166.751734 106.425266) (width 0.1524) (layer F.Cu) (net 8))
 (segment (start 140.208 105.4735) (end 140.9065 105.4735) (width 0.1524) (layer B.Cu) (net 8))
 (segment (start 137.541 102.8065) (end 140.208 105.4735) (width 0.1524) (layer B.Cu) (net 8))
 (via (at 140.9065 105.4735) (size 0.6) (drill 0.4) (layers F.Cu B.Cu) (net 8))
 (segment (start 137.541 97.4725) (end 137.541 102.8065) (width 0.1524) (layer B.Cu) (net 8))
 (segment (start 137.541 93.7895) (end 137.541 97.4725) (width 0.1524) (layer F.Cu) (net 8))
 (via (at 137.541 97.4725) (size 0.6) (drill 0.4) (layers F.Cu B.Cu) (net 8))
 (segment (start 135.961734 92.210234) (end 137.541 93.7895) (width 0.1524) (layer F.Cu) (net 8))
 (segment (start 135.961734 90.324098) (end 135.961734 92.210234) (width 0.1524) (layer F.Cu) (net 8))
 (segment (start 166.751734 102.762098) (end 166.751734 104.162098) (width 0.2) (layer F.Cu) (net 8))
 (segment (start 169.037734 98.526098) (end 169.037734 101.046098) (width 0.2) (layer F.Cu) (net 8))
 (segment (start 169.037734 101.046098) (end 167.321734 102.762098) (width 0.2) (layer F.Cu) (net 8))
 (segment (start 167.321734 102.762098) (end 166.751734 102.762098) (width 0.2) (layer F.Cu) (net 8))
 (segment (start 170.815734 96.748098) (end 169.037734 98.526098) (width 0.2) (layer F.Cu) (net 8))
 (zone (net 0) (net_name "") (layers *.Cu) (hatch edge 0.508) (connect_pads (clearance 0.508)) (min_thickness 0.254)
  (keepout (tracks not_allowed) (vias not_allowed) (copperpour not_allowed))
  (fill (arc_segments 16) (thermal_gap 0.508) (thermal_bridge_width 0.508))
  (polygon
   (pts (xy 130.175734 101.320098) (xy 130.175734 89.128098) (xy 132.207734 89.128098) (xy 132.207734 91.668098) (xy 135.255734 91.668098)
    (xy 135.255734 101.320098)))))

